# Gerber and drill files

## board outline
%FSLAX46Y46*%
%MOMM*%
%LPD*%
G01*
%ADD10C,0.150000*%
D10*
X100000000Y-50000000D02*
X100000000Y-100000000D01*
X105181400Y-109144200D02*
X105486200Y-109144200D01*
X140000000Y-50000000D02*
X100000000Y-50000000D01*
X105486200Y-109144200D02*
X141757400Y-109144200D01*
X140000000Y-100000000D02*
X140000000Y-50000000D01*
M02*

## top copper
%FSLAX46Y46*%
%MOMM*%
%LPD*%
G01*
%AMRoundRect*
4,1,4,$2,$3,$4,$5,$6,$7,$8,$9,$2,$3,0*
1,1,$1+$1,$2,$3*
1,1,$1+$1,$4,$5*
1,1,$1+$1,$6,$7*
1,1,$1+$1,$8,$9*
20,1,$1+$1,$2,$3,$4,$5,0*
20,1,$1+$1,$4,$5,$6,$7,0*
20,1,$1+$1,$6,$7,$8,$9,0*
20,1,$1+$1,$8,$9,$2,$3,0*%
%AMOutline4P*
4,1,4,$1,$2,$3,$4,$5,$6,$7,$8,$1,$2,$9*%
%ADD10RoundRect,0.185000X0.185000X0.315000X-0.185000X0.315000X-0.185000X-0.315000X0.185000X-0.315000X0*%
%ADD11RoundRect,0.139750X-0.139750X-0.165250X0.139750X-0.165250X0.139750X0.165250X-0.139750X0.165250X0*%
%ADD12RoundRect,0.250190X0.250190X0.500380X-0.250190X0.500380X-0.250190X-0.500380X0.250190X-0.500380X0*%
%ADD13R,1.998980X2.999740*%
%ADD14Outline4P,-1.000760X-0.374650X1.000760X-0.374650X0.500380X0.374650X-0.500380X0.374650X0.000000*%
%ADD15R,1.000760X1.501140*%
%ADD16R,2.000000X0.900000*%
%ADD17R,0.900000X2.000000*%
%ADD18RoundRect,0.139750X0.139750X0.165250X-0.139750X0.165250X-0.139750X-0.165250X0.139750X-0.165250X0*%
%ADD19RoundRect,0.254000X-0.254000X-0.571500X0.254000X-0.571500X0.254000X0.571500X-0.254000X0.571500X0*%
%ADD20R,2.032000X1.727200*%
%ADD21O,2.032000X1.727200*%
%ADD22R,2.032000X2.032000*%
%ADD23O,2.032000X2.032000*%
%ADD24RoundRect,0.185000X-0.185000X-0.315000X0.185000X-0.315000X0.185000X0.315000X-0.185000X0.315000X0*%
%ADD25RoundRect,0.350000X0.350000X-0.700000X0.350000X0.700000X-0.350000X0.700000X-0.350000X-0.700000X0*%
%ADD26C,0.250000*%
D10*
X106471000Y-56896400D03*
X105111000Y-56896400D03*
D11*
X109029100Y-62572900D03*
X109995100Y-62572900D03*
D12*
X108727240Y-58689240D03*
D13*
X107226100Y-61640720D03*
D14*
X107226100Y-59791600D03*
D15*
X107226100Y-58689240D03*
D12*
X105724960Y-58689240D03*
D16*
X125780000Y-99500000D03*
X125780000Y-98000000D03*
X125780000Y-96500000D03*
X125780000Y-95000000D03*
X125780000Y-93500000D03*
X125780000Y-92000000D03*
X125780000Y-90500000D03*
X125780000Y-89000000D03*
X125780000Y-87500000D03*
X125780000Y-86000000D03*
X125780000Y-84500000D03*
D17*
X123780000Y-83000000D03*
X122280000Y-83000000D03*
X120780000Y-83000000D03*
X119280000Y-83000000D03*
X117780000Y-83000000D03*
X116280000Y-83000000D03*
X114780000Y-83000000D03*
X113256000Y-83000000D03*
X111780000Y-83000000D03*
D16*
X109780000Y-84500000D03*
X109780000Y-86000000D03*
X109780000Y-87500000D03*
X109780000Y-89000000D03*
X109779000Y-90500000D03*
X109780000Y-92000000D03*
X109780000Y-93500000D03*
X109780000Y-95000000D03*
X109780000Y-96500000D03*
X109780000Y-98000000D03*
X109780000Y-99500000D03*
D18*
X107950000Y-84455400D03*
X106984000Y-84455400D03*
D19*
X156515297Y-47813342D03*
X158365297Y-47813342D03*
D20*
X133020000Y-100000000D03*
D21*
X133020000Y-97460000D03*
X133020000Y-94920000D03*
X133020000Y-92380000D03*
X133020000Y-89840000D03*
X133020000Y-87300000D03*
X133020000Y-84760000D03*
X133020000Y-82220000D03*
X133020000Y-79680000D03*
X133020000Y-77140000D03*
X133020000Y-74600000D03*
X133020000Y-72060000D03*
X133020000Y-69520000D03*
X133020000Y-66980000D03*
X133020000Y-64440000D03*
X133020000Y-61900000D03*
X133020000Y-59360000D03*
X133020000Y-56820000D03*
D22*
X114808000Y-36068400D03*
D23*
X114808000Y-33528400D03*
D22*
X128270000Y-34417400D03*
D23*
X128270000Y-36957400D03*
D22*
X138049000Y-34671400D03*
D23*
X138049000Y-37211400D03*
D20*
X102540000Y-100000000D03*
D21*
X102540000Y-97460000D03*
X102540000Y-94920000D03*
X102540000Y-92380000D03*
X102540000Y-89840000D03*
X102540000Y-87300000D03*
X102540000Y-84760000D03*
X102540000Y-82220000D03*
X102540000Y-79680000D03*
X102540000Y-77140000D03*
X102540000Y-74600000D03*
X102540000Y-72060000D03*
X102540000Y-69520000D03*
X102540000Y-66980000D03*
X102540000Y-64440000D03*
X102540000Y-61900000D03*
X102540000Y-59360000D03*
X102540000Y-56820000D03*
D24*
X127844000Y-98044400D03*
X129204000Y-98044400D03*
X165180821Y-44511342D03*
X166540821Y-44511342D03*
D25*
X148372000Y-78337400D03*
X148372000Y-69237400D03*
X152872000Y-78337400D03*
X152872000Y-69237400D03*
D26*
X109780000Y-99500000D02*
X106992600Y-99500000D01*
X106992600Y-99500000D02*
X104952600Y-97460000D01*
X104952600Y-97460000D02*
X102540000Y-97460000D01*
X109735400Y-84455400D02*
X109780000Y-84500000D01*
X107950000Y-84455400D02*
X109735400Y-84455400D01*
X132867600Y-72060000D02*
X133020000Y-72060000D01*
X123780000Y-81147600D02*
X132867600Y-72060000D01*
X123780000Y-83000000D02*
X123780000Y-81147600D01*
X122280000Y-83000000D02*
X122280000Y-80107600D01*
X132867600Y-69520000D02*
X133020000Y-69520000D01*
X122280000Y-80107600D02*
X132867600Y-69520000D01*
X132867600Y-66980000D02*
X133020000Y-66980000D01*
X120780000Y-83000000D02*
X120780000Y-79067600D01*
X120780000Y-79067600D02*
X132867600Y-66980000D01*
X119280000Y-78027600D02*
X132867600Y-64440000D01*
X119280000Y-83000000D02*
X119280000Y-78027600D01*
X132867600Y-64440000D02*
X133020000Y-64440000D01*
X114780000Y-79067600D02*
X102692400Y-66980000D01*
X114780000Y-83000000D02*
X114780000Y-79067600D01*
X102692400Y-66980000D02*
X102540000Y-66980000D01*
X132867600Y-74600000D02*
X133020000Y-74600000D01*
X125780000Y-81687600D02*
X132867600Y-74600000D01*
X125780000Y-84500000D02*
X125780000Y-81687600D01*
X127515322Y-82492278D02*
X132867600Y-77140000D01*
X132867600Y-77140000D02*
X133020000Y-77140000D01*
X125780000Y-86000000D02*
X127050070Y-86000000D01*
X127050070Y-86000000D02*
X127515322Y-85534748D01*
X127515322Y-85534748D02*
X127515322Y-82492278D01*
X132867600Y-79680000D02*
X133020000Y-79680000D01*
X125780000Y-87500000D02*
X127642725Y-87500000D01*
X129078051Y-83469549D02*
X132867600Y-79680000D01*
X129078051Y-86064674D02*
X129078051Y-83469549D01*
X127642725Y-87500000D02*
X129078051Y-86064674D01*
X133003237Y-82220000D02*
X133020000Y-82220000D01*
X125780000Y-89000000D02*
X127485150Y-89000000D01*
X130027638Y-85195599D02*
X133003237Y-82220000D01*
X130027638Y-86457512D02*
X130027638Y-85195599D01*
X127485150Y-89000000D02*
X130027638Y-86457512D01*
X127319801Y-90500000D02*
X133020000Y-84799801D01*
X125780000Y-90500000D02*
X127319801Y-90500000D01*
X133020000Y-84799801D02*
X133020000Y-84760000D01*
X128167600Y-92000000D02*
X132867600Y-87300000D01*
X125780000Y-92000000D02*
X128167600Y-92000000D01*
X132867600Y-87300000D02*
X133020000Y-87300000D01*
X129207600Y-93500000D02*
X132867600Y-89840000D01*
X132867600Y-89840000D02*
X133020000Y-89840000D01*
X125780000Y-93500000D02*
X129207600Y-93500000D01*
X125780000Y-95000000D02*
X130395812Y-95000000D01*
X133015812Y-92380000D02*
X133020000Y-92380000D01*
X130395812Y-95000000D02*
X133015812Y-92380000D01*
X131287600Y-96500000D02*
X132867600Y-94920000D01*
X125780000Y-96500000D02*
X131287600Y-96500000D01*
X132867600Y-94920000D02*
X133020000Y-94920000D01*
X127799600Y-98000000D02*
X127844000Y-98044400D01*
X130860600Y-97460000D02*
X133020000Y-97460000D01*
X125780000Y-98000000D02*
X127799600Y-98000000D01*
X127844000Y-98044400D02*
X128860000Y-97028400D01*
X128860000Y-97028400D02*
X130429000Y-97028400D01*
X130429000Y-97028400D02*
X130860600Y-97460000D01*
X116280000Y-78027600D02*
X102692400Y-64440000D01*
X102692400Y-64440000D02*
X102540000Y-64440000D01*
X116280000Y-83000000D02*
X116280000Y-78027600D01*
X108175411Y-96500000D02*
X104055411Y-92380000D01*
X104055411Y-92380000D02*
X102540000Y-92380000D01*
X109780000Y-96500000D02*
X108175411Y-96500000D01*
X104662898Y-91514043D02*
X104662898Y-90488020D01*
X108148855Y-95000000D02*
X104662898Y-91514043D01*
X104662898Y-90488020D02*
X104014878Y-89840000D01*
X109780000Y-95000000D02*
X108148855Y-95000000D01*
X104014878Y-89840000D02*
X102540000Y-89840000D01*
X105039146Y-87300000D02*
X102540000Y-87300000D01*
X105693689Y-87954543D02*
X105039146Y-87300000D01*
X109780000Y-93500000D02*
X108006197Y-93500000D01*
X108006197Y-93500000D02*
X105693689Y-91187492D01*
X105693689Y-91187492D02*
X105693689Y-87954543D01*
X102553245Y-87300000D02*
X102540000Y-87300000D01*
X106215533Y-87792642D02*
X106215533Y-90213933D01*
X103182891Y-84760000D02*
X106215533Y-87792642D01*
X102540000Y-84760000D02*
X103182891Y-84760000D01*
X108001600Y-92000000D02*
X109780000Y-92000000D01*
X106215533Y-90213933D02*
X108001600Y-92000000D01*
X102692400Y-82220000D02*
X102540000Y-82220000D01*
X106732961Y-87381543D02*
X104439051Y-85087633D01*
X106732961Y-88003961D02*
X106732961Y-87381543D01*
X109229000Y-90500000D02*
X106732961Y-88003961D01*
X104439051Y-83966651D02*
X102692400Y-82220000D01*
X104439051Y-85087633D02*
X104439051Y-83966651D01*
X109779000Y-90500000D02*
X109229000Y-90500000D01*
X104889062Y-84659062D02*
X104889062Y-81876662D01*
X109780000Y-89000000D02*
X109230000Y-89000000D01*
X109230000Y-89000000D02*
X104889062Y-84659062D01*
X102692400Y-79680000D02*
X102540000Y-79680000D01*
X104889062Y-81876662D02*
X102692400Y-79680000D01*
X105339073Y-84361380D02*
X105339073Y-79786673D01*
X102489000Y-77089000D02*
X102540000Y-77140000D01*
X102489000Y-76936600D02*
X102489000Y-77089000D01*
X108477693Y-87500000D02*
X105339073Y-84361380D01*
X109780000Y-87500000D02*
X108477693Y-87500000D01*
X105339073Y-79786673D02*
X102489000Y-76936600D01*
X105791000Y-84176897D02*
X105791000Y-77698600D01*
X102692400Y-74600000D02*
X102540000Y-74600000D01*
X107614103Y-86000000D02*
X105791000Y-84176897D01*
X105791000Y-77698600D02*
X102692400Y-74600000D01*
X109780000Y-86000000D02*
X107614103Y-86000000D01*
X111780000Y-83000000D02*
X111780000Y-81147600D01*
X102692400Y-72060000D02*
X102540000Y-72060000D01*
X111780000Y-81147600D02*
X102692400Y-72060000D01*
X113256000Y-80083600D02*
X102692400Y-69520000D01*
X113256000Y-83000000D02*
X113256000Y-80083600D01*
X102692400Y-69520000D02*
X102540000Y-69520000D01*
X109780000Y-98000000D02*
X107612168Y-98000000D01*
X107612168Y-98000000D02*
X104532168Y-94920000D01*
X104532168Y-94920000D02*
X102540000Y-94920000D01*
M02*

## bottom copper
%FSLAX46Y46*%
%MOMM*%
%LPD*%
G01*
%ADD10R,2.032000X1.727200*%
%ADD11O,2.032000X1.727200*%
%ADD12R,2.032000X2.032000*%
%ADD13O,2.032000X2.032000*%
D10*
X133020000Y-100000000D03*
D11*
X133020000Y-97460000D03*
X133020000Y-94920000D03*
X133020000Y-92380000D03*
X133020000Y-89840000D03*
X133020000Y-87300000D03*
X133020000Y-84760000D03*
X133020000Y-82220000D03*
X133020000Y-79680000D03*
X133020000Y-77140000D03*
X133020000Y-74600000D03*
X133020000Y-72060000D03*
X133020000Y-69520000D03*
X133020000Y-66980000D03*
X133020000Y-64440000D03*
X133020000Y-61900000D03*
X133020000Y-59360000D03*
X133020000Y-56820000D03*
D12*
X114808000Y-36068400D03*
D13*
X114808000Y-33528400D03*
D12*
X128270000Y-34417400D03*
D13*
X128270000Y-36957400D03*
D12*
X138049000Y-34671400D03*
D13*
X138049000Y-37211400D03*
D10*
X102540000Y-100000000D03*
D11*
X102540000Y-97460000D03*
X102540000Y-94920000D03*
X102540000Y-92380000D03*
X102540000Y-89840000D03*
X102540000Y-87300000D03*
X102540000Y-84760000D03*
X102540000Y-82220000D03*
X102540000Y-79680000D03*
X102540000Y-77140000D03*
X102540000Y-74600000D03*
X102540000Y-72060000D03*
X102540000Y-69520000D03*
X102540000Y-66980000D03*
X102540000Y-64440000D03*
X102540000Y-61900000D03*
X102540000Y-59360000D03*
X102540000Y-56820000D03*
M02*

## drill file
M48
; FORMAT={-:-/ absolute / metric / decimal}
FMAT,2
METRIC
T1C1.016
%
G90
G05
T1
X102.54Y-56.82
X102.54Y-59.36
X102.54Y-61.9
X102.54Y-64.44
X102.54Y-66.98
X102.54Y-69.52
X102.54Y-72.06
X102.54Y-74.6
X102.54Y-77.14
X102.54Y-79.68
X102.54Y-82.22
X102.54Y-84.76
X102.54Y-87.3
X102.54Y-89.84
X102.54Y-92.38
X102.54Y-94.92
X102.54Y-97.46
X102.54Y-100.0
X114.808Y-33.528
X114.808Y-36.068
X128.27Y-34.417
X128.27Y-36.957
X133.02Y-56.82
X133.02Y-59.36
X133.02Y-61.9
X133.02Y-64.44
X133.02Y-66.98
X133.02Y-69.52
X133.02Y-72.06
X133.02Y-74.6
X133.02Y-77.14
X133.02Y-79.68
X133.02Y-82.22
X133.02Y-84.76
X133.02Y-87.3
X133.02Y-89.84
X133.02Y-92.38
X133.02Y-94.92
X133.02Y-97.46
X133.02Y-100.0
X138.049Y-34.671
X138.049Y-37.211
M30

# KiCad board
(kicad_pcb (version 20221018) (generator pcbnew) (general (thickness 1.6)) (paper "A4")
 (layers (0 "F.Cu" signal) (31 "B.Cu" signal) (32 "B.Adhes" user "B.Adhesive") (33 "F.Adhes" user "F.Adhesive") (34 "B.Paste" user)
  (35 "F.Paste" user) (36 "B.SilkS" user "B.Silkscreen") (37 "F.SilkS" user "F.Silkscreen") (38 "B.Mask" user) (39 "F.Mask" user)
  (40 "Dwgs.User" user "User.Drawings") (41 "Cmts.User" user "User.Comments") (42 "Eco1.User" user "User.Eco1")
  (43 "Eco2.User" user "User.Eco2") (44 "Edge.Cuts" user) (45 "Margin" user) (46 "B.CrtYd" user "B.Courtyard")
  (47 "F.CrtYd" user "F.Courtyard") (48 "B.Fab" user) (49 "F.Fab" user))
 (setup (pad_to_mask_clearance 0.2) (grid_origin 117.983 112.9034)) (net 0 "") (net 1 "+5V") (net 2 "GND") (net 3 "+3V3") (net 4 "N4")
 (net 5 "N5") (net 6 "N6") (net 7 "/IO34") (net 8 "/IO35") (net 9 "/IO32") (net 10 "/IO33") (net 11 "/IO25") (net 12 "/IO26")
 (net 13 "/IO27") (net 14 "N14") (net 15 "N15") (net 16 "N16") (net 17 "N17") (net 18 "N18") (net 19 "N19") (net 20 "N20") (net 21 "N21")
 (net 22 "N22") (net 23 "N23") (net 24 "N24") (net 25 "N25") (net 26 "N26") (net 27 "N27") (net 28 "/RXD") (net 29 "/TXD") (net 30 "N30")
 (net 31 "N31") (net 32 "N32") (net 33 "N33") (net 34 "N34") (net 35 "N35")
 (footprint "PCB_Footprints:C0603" (layer "F.Cu") (at 105.791 56.8964 180)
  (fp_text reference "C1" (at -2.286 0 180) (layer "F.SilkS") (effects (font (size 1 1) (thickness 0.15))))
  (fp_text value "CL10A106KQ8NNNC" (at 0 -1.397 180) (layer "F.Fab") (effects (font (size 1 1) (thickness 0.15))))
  (pad "1" smd roundrect (at -0.68 0 180) (size 0.74 1) (layers "F.Cu" "F.Paste" "F.Mask") (roundrect_rratio 0.25) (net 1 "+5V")
   (solder_mask_margin 0.102))
  (pad "2" smd roundrect (at 0.68 0 180) (size 0.74 1) (layers "F.Cu" "F.Paste" "F.Mask") (roundrect_rratio 0.25) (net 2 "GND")
   (solder_mask_margin 0.102)))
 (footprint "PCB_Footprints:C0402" (layer "F.Cu") (at 109.5121 62.5729)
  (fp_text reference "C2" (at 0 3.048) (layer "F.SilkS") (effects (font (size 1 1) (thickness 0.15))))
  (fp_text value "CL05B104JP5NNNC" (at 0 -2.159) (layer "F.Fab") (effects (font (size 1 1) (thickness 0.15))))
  (pad "1" smd roundrect (at -0.483 0) (size 0.559 0.61) (layers "F.Cu" "F.Paste" "F.Mask") (roundrect_rratio 0.25) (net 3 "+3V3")
   (solder_mask_margin 0.102))
  (pad "2" smd roundrect (at 0.483 0) (size 0.559 0.61) (layers "F.Cu" "F.Paste" "F.Mask") (roundrect_rratio 0.25) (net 2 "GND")
   (solder_mask_margin 0.102)))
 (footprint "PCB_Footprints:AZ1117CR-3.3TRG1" (layer "F.Cu") (at 107.2261 60.5409 180)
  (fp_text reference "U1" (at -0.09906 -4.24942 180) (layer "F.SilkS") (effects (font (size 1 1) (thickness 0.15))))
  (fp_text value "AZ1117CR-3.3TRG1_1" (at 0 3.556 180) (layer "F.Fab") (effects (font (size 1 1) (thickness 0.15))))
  (pad "1" smd roundrect (at -1.50114 1.85166 180) (size 1.00076 1.50114) (layers "F.Cu" "F.Paste" "F.Mask") (roundrect_rratio 0.25)
   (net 2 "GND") (solder_mask_margin 0.102))
  (pad "2" smd rect (at 0 -1.09982 180) (size 1.99898 2.99974) (layers "F.Cu" "F.Paste" "F.Mask") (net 3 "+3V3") (solder_mask_margin 0.102))
  (pad "2" smd trapezoid (at 0 0.7493) (size 1.50114 0.7493) (rect_delta 0 0.50038) (layers "F.Cu" "F.Paste" "F.Mask") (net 3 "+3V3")
   (solder_mask_margin 0.102))
  (pad "2" smd rect (at 0 1.85166 180) (size 1.00076 1.50114) (layers "F.Cu" "F.Paste" "F.Mask") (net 3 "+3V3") (solder_mask_margin 0.102))
  (pad "3" smd roundrect (at 1.50114 1.85166 180) (size 1.00076 1.50114) (layers "F.Cu" "F.Paste" "F.Mask") (roundrect_rratio 0.25)
   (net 1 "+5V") (solder_mask_margin 0.102)))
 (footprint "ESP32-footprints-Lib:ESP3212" (layer "F.Cu") (at 117.78 95 180)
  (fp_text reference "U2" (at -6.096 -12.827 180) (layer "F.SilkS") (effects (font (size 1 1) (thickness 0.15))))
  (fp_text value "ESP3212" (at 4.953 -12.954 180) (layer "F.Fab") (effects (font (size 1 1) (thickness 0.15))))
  (pad "1" smd rect (at -8 -4.5 180) (size 2 0.9) (layers "F.Cu" "F.Paste" "F.Mask") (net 2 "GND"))
  (pad "2" smd rect (at -8 -3 180) (size 2 0.9) (layers "F.Cu" "F.Paste" "F.Mask") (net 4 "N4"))
  (pad "3" smd rect (at -8 -1.5 180) (size 2 0.9) (layers "F.Cu" "F.Paste" "F.Mask") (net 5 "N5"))
  (pad "4" smd rect (at -8 0 180) (size 2 0.9) (layers "F.Cu" "F.Paste" "F.Mask") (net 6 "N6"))
  (pad "5" smd rect (at -8 1.5 180) (size 2 0.9) (layers "F.Cu" "F.Paste" "F.Mask") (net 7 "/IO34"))
  (pad "6" smd rect (at -8 3 180) (size 2 0.9) (layers "F.Cu" "F.Paste" "F.Mask") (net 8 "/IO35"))
  (pad "7" smd rect (at -8 4.5 180) (size 2 0.9) (layers "F.Cu" "F.Paste" "F.Mask") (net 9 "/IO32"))
  (pad "8" smd rect (at -8 6 180) (size 2 0.9) (layers "F.Cu" "F.Paste" "F.Mask") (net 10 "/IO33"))
  (pad "9" smd rect (at -8 7.5 180) (size 2 0.9) (layers "F.Cu" "F.Paste" "F.Mask") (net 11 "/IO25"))
  (pad "10" smd rect (at -8 9 180) (size 2 0.9) (layers "F.Cu" "F.Paste" "F.Mask") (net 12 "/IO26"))
  (pad "11" smd rect (at -8 10.5 180) (size 2 0.9) (layers "F.Cu" "F.Paste" "F.Mask") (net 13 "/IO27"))
  (pad "12" smd rect (at -6 12 180) (size 0.9 2) (layers "F.Cu" "F.Paste" "F.Mask") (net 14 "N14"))
  (pad "13" smd rect (at -4.5 12 180) (size 0.9 2) (layers "F.Cu" "F.Paste" "F.Mask") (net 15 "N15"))
  (pad "14" smd rect (at -3 12 180) (size 0.9 2) (layers "F.Cu" "F.Paste" "F.Mask") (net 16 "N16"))
  (pad "15" smd rect (at -1.5 12 180) (size 0.9 2) (layers "F.Cu" "F.Paste" "F.Mask") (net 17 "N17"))
  (pad "16" smd rect (at 0 12 180) (size 0.9 2) (layers "F.Cu" "F.Paste" "F.Mask") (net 2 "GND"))
  (pad "17" smd rect (at 1.5 12 180) (size 0.9 2) (layers "F.Cu" "F.Paste" "F.Mask") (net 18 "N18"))
  (pad "18" smd rect (at 3 12 180) (size 0.9 2) (layers "F.Cu" "F.Paste" "F.Mask") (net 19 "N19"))
  (pad "19" smd rect (at 4.524 12 180) (size 0.9 2) (layers "F.Cu" "F.Paste" "F.Mask") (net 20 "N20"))
  (pad "20" smd rect (at 6 12 180) (size 0.9 2) (layers "F.Cu" "F.Paste" "F.Mask") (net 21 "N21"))
  (pad "21" smd rect (at 8 10.5 180) (size 2 0.9) (layers "F.Cu" "F.Paste" "F.Mask") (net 3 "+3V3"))
  (pad "22" smd rect (at 8 9 180) (size 2 0.9) (layers "F.Cu" "F.Paste" "F.Mask") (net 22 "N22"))
  (pad "23" smd rect (at 8 7.5 180) (size 2 0.9) (layers "F.Cu" "F.Paste" "F.Mask") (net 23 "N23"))
  (pad "24" smd rect (at 8 6 180) (size 2 0.9) (layers "F.Cu" "F.Paste" "F.Mask") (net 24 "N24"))
  (pad "25" smd rect (at 8.001 4.5 180) (size 2 0.9) (layers "F.Cu" "F.Paste" "F.Mask") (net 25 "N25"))
  (pad "26" smd rect (at 8 3 180) (size 2 0.9) (layers "F.Cu" "F.Paste" "F.Mask") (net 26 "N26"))
  (pad "27" smd rect (at 8 1.5 180) (size 2 0.9) (layers "F.Cu" "F.Paste" "F.Mask") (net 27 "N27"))
  (pad "28" smd rect (at 8 0 180) (size 2 0.9) (layers "F.Cu" "F.Paste" "F.Mask") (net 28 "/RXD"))
  (pad "29" smd rect (at 8 -1.5 180) (size 2 0.9) (layers "F.Cu" "F.Paste" "F.Mask") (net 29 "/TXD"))
  (pad "30" smd rect (at 8 -3 180) (size 2 0.9) (layers "F.Cu" "F.Paste" "F.Mask") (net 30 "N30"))
  (pad "31" smd rect (at 8 -4.5 180) (size 2 0.9) (layers "F.Cu" "F.Paste" "F.Mask") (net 2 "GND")))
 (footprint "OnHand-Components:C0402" (layer "F.Cu") (at 107.467 84.4554 180)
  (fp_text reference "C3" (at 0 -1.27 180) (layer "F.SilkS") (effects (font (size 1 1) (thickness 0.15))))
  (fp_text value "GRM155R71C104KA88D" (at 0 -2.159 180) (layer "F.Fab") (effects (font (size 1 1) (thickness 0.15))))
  (pad "1" smd roundrect (at -0.483 0 180) (size 0.559 0.61) (layers "F.Cu" "F.Paste" "F.Mask") (roundrect_rratio 0.25) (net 3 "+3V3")
   (solder_mask_margin 0.102))
  (pad "2" smd roundrect (at 0.483 0 180) (size 0.559 0.61) (layers "F.Cu" "F.Paste" "F.Mask") (roundrect_rratio 0.25) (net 2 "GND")
   (solder_mask_margin 0.102)))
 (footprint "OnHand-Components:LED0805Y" (layer "F.Cu") (at 157.440297 47.813342)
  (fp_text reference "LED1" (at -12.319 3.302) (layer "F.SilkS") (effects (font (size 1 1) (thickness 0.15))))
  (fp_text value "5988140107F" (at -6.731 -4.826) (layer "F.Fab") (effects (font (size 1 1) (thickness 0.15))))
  (pad "1" smd roundrect (at -0.925 0) (size 1.016 1.651) (layers "F.Cu" "F.Paste" "F.Mask") (roundrect_rratio 0.25) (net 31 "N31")
   (solder_mask_margin 0.102))
  (pad "2" smd roundrect (at 0.925 0) (size 1.016 1.651) (layers "F.Cu" "F.Paste" "F.Mask") (roundrect_rratio 0.25) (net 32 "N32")
   (solder_mask_margin 0.102)))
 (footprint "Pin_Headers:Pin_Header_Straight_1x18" (layer "F.Cu") (at 133.02 100 180)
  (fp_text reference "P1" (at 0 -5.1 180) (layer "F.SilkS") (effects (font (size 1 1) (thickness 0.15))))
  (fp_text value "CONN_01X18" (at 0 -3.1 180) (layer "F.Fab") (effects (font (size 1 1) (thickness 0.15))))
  (pad "1" thru_hole rect (at 0 0 180) (size 2.032 1.7272) (drill 1.016) (layers "*.Cu" "*.Mask" "F.SilkS") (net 2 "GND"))
  (pad "2" thru_hole oval (at 0 2.54 180) (size 2.032 1.7272) (drill 1.016) (layers "*.Cu" "*.Mask" "F.SilkS") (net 4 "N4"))
  (pad "3" thru_hole oval (at 0 5.08 180) (size 2.032 1.7272) (drill 1.016) (layers "*.Cu" "*.Mask" "F.SilkS") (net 5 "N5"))
  (pad "4" thru_hole oval (at 0 7.62 180) (size 2.032 1.7272) (drill 1.016) (layers "*.Cu" "*.Mask" "F.SilkS") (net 6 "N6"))
  (pad "5" thru_hole oval (at 0 10.16 180) (size 2.032 1.7272) (drill 1.016) (layers "*.Cu" "*.Mask" "F.SilkS") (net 7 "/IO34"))
  (pad "6" thru_hole oval (at 0 12.7 180) (size 2.032 1.7272) (drill 1.016) (layers "*.Cu" "*.Mask" "F.SilkS") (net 8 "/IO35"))
  (pad "7" thru_hole oval (at 0 15.24 180) (size 2.032 1.7272) (drill 1.016) (layers "*.Cu" "*.Mask" "F.SilkS") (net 9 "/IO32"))
  (pad "8" thru_hole oval (at 0 17.78 180) (size 2.032 1.7272) (drill 1.016) (layers "*.Cu" "*.Mask" "F.SilkS") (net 10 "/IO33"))
  (pad "9" thru_hole oval (at 0 20.32 180) (size 2.032 1.7272) (drill 1.016) (layers "*.Cu" "*.Mask" "F.SilkS") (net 11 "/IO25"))
  (pad "10" thru_hole oval (at 0 22.86 180) (size 2.032 1.7272) (drill 1.016) (layers "*.Cu" "*.Mask" "F.SilkS") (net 12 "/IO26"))
  (pad "11" thru_hole oval (at 0 25.4 180) (size 2.032 1.7272) (drill 1.016) (layers "*.Cu" "*.Mask" "F.SilkS") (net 13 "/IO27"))
  (pad "12" thru_hole oval (at 0 27.94 180) (size 2.032 1.7272) (drill 1.016) (layers "*.Cu" "*.Mask" "F.SilkS") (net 14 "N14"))
  (pad "13" thru_hole oval (at 0 30.48 180) (size 2.032 1.7272) (drill 1.016) (layers "*.Cu" "*.Mask" "F.SilkS") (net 15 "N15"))
  (pad "14" thru_hole oval (at 0 33.02 180) (size 2.032 1.7272) (drill 1.016) (layers "*.Cu" "*.Mask" "F.SilkS") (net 16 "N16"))
  (pad "15" thru_hole oval (at 0 35.56 180) (size 2.032 1.7272) (drill 1.016) (layers "*.Cu" "*.Mask" "F.SilkS") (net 17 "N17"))
  (pad "16" thru_hole oval (at 0 38.1 180) (size 2.032 1.7272) (drill 1.016) (layers "*.Cu" "*.Mask" "F.SilkS") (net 3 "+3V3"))
  (pad "17" thru_hole oval (at 0 40.64 180) (size 2.032 1.7272) (drill 1.016) (layers "*.Cu" "*.Mask" "F.SilkS") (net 1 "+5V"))
  (pad "18" thru_hole oval (at 0 43.18 180) (size 2.032 1.7272) (drill 1.016) (layers "*.Cu" "*.Mask" "F.SilkS") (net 2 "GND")))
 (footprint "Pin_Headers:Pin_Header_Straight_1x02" (layer "F.Cu") (at 114.808 36.0684 180)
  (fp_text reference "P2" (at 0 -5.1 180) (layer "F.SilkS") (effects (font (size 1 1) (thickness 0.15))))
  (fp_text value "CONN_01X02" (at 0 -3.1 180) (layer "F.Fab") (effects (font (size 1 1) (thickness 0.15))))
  (pad "1" thru_hole rect (at 0 0 180) (size 2.032 2.032) (drill 1.016) (layers "*.Cu" "*.Mask" "F.SilkS") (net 19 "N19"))
  (pad "2" thru_hole oval (at 0 2.54 180) (size 2.032 2.032) (drill 1.016) (layers "*.Cu" "*.Mask" "F.SilkS") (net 2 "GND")))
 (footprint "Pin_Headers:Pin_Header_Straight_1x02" (layer "F.Cu") (at 128.27 34.4174)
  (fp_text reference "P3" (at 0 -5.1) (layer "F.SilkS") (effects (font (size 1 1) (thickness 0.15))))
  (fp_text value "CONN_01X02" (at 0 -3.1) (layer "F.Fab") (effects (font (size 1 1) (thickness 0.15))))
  (pad "1" thru_hole rect (at 0 0) (size 2.032 2.032) (drill 1.016) (layers "*.Cu" "*.Mask" "F.SilkS") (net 18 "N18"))
  (pad "2" thru_hole oval (at 0 2.54) (size 2.032 2.032) (drill 1.016) (layers "*.Cu" "*.Mask" "F.SilkS") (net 2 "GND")))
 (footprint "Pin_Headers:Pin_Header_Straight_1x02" (layer "F.Cu") (at 138.049 34.6714)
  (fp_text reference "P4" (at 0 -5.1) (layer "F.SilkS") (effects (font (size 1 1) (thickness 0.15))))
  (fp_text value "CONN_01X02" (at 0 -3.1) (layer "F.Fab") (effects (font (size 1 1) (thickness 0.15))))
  (pad "1" thru_hole rect (at 0 0) (size 2.032 2.032) (drill 1.016) (layers "*.Cu" "*.Mask" "F.SilkS") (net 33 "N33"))
  (pad "2" thru_hole oval (at 0 2.54) (size 2.032 2.032) (drill 1.016) (layers "*.Cu" "*.Mask" "F.SilkS") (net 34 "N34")))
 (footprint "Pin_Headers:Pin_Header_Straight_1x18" (layer "F.Cu") (at 102.54 100 180)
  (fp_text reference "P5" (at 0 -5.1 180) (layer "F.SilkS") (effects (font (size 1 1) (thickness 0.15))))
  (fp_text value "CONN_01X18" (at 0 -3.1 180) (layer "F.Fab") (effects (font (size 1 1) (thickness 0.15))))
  (pad "1" thru_hole rect (at 0 0 180) (size 2.032 1.7272) (drill 1.016) (layers "*.Cu" "*.Mask" "F.SilkS") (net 2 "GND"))
  (pad "2" thru_hole oval (at 0 2.54 180) (size 2.032 1.7272) (drill 1.016) (layers "*.Cu" "*.Mask" "F.SilkS") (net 2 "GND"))
  (pad "3" thru_hole oval (at 0 5.08 180) (size 2.032 1.7272) (drill 1.016) (layers "*.Cu" "*.Mask" "F.SilkS") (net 30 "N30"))
  (pad "4" thru_hole oval (at 0 7.62 180) (size 2.032 1.7272) (drill 1.016) (layers "*.Cu" "*.Mask" "F.SilkS") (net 29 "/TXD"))
  (pad "5" thru_hole oval (at 0 10.16 180) (size 2.032 1.7272) (drill 1.016) (layers "*.Cu" "*.Mask" "F.SilkS") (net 28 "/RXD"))
  (pad "6" thru_hole oval (at 0 12.7 180) (size 2.032 1.7272) (drill 1.016) (layers "*.Cu" "*.Mask" "F.SilkS") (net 27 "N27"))
  (pad "7" thru_hole oval (at 0 15.24 180) (size 2.032 1.7272) (drill 1.016) (layers "*.Cu" "*.Mask" "F.SilkS") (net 26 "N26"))
  (pad "8" thru_hole oval (at 0 17.78 180) (size 2.032 1.7272) (drill 1.016) (layers "*.Cu" "*.Mask" "F.SilkS") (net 25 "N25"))
  (pad "9" thru_hole oval (at 0 20.32 180) (size 2.032 1.7272) (drill 1.016) (layers "*.Cu" "*.Mask" "F.SilkS") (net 24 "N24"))
  (pad "10" thru_hole oval (at 0 22.86 180) (size 2.032 1.7272) (drill 1.016) (layers "*.Cu" "*.Mask" "F.SilkS") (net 23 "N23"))
  (pad "11" thru_hole oval (at 0 25.4 180) (size 2.032 1.7272) (drill 1.016) (layers "*.Cu" "*.Mask" "F.SilkS") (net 22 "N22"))
  (pad "12" thru_hole oval (at 0 27.94 180) (size 2.032 1.7272) (drill 1.016) (layers "*.Cu" "*.Mask" "F.SilkS") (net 21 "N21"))
  (pad "13" thru_hole oval (at 0 30.48 180) (size 2.032 1.7272) (drill 1.016) (layers "*.Cu" "*.Mask" "F.SilkS") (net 20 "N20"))
  (pad "14" thru_hole oval (at 0 33.02 180) (size 2.032 1.7272) (drill 1.016) (layers "*.Cu" "*.Mask" "F.SilkS") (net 19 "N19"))
  (pad "15" thru_hole oval (at 0 35.56 180) (size 2.032 1.7272) (drill 1.016) (layers "*.Cu" "*.Mask" "F.SilkS") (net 18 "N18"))
  (pad "16" thru_hole oval (at 0 38.1 180) (size 2.032 1.7272) (drill 1.016) (layers "*.Cu" "*.Mask" "F.SilkS") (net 3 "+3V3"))
  (pad "17" thru_hole oval (at 0 40.64 180) (size 2.032 1.7272) (drill 1.016) (layers "*.Cu" "*.Mask" "F.SilkS") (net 1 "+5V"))
  (pad "18" thru_hole oval (at 0 43.18 180) (size 2.032 1.7272) (drill 1.016) (layers "*.Cu" "*.Mask" "F.SilkS") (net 2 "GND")))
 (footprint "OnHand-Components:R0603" (layer "F.Cu") (at 128.524 98.0444)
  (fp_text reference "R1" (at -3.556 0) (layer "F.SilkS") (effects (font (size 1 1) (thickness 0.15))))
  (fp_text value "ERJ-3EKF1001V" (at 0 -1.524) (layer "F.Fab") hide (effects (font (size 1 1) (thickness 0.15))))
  (pad "1" smd roundrect (at -0.68 0) (size 0.74 1) (layers "F.Cu" "F.Paste" "F.Mask") (roundrect_rratio 0.25) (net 4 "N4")
   (solder_mask_margin 0.102))
  (pad "2" smd roundrect (at 0.68 0) (size 0.74 1) (layers "F.Cu" "F.Paste" "F.Mask") (roundrect_rratio 0.25) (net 3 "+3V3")
   (solder_mask_margin 0.102)))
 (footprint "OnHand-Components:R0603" (layer "F.Cu") (at 165.860821 44.511342)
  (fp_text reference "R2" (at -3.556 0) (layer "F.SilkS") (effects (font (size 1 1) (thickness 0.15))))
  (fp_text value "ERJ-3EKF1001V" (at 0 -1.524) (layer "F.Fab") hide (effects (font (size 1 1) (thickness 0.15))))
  (pad "1" smd roundrect (at -0.68 0) (size 0.74 1) (layers "F.Cu" "F.Paste" "F.Mask") (roundrect_rratio 0.25) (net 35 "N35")
   (solder_mask_margin 0.102))
  (pad "2" smd roundrect (at 0.68 0) (size 0.74 1) (layers "F.Cu" "F.Paste" "F.Mask") (roundrect_rratio 0.25) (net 33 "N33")
   (solder_mask_margin 0.102)))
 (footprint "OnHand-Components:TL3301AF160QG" (layer "F.Cu") (at 150.622 73.7874 90)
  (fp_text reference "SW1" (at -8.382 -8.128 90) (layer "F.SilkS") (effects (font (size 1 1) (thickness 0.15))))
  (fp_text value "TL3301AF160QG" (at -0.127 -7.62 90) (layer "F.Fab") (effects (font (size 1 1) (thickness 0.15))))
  (pad "1" smd roundrect (at -4.55 -2.25 90) (size 2.1 1.4) (layers "F.Cu" "F.Paste" "F.Mask") (roundrect_rratio 0.25) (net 2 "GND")
   (solder_mask_margin 0.102))
  (pad "1" smd roundrect (at 4.55 -2.25 90) (size 2.1 1.4) (layers "F.Cu" "F.Paste" "F.Mask") (roundrect_rratio 0.25) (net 2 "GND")
   (solder_mask_margin 0.102))
  (pad "2" smd roundrect (at -4.55 2.25 90) (size 2.1 1.4) (layers "F.Cu" "F.Paste" "F.Mask") (roundrect_rratio 0.25) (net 4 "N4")
   (solder_mask_margin 0.102))
  (pad "2" smd roundrect (at 4.55 2.25 90) (size 2.1 1.4) (layers "F.Cu" "F.Paste" "F.Mask") (roundrect_rratio 0.25) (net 4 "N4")
   (solder_mask_margin 0.102)))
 (gr_line (start 100 50) (end 100 100) (stroke (width 0.15) (type solid)) (layer "Edge.Cuts"))
 (gr_line (start 105.1814 109.1442) (end 105.4862 109.1442) (stroke (width 0.15) (type solid)) (layer "Edge.Cuts"))
 (gr_line (start 140 50) (end 100 50) (stroke (width 0.15) (type solid)) (layer "Edge.Cuts"))
 (gr_line (start 105.4862 109.1442) (end 141.7574 109.1442) (stroke (width 0.15) (type solid)) (layer "Edge.Cuts"))
 (gr_line (start 140 100) (end 140 50) (stroke (width 0.15) (type solid)) (layer "Edge.Cuts"))
 (segment (start 109.78 99.5) (end 106.9926 99.5) (width 0.25) (layer "F.Cu") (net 2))
 (segment (start 106.9926 99.5) (end 104.9526 97.46) (width 0.25) (layer "F.Cu") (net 2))
 (segment (start 104.9526 97.46) (end 102.54 97.46) (width 0.25) (layer "F.Cu") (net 2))
 (segment (start 109.7354 84.4554) (end 109.78 84.5) (width 0.25) (layer "F.Cu") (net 3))
 (segment (start 107.95 84.4554) (end 109.7354 84.4554) (width 0.25) (layer "F.Cu") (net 3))
 (segment (start 132.8676 72.06) (end 133.02 72.06) (width 0.25) (layer "F.Cu") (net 14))
 (segment (start 123.78 81.1476) (end 132.8676 72.06) (width 0.25) (layer "F.Cu") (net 14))
 (segment (start 123.78 83) (end 123.78 81.1476) (width 0.25) (layer "F.Cu") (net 14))
 (segment (start 122.28 83) (end 122.28 80.1076) (width 0.25) (layer "F.Cu") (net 15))
 (segment (start 132.8676 69.52) (end 133.02 69.52) (width 0.25) (layer "F.Cu") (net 15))
 (segment (start 122.28 80.1076) (end 132.8676 69.52) (width 0.25) (layer "F.Cu") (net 15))
 (segment (start 132.8676 66.98) (end 133.02 66.98) (width 0.25) (layer "F.Cu") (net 16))
 (segment (start 120.78 83) (end 120.78 79.0676) (width 0.25) (layer "F.Cu") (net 16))
 (segment (start 120.78 79.0676) (end 132.8676 66.98) (width 0.25) (layer "F.Cu") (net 16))
 (segment (start 119.28 78.0276) (end 132.8676 64.44) (width 0.25) (layer "F.Cu") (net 17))
 (segment (start 119.28 83) (end 119.28 78.0276) (width 0.25) (layer "F.Cu") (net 17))
 (segment (start 132.8676 64.44) (end 133.02 64.44) (width 0.25) (layer "F.Cu") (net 17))
 (segment (start 114.78 79.0676) (end 102.6924 66.98) (width 0.25) (layer "F.Cu") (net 19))
 (segment (start 114.78 83) (end 114.78 79.0676) (width 0.25) (layer "F.Cu") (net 19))
 (segment (start 102.6924 66.98) (end 102.54 66.98) (width 0.25) (layer "F.Cu") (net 19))
 (segment (start 132.8676 74.6) (end 133.02 74.6) (width 0.25) (layer "F.Cu") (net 13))
 (segment (start 125.78 81.6876) (end 132.8676 74.6) (width 0.25) (layer "F.Cu") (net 13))
 (segment (start 125.78 84.5) (end 125.78 81.6876) (width 0.25) (layer "F.Cu") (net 13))
 (segment (start 127.515322 82.492278) (end 132.8676 77.14) (width 0.25) (layer "F.Cu") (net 12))
 (segment (start 132.8676 77.14) (end 133.02 77.14) (width 0.25) (layer "F.Cu") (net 12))
 (segment (start 125.78 86) (end 127.05007 86) (width 0.25) (layer "F.Cu") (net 12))
 (segment (start 127.05007 86) (end 127.515322 85.534748) (width 0.25) (layer "F.Cu") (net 12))
 (segment (start 127.515322 85.534748) (end 127.515322 82.492278) (width 0.25) (layer "F.Cu") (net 12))
 (segment (start 132.8676 79.68) (end 133.02 79.68) (width 0.25) (layer "F.Cu") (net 11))
 (segment (start 125.78 87.5) (end 127.642725 87.5) (width 0.25) (layer "F.Cu") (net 11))
 (segment (start 129.078051 83.469549) (end 132.8676 79.68) (width 0.25) (layer "F.Cu") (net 11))
 (segment (start 129.078051 86.064674) (end 129.078051 83.469549) (width 0.25) (layer "F.Cu") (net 11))
 (segment (start 127.642725 87.5) (end 129.078051 86.064674) (width 0.25) (layer "F.Cu") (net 11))
 (segment (start 133.003237 82.22) (end 133.02 82.22) (width 0.25) (layer "F.Cu") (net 10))
 (segment (start 125.78 89) (end 127.48515 89) (width 0.25) (layer "F.Cu") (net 10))
 (segment (start 130.027638 85.195599) (end 133.003237 82.22) (width 0.25) (layer "F.Cu") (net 10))
 (segment (start 130.027638 86.457512) (end 130.027638 85.195599) (width 0.25) (layer "F.Cu") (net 10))
 (segment (start 127.48515 89) (end 130.027638 86.457512) (width 0.25) (layer "F.Cu") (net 10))
 (segment (start 127.319801 90.5) (end 133.02 84.799801) (width 0.25) (layer "F.Cu") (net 9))
 (segment (start 125.78 90.5) (end 127.319801 90.5) (width 0.25) (layer "F.Cu") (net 9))
 (segment (start 133.02 84.799801) (end 133.02 84.76) (width 0.25) (layer "F.Cu") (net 9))
 (segment (start 128.1676 92) (end 132.8676 87.3) (width 0.25) (layer "F.Cu") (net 8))
 (segment (start 125.78 92) (end 128.1676 92) (width 0.25) (layer "F.Cu") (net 8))
 (segment (start 132.8676 87.3) (end 133.02 87.3) (width 0.25) (layer "F.Cu") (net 8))
 (segment (start 129.2076 93.5) (end 132.8676 89.84) (width 0.25) (layer "F.Cu") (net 7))
 (segment (start 132.8676 89.84) (end 133.02 89.84) (width 0.25) (layer "F.Cu") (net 7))
 (segment (start 125.78 93.5) (end 129.2076 93.5) (width 0.25) (layer "F.Cu") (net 7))
 (segment (start 125.78 95) (end 130.395812 95) (width 0.25) (layer "F.Cu") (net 6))
 (segment (start 133.015812 92.38) (end 133.02 92.38) (width 0.25) (layer "F.Cu") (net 6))
 (segment (start 130.395812 95) (end 133.015812 92.38) (width 0.25) (layer "F.Cu") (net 6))
 (segment (start 131.2876 96.5) (end 132.8676 94.92) (width 0.25) (layer "F.Cu") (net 5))
 (segment (start 125.78 96.5) (end 131.2876 96.5) (width 0.25) (layer "F.Cu") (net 5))
 (segment (start 132.8676 94.92) (end 133.02 94.92) (width 0.25) (layer "F.Cu") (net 5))
 (segment (start 127.7996 98) (end 127.844 98.0444) (width 0.25) (layer "F.Cu") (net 4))
 (segment (start 130.8606 97.46) (end 133.02 97.46) (width 0.25) (layer "F.Cu") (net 4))
 (segment (start 125.78 98) (end 127.7996 98) (width 0.25) (layer "F.Cu") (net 4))
 (segment (start 127.844 98.0444) (end 128.86 97.0284) (width 0.25) (layer "F.Cu") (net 4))
 (segment (start 128.86 97.0284) (end 130.429 97.0284) (width 0.25) (layer "F.Cu") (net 4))
 (segment (start 130.429 97.0284) (end 130.8606 97.46) (width 0.25) (layer "F.Cu") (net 4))
 (segment (start 116.28 78.0276) (end 102.6924 64.44) (width 0.25) (layer "F.Cu") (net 18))
 (segment (start 102.6924 64.44) (end 102.54 64.44) (width 0.25) (layer "F.Cu") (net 18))
 (segment (start 116.28 83) (end 116.28 78.0276) (width 0.25) (layer "F.Cu") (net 18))
 (segment (start 108.175411 96.5) (end 104.055411 92.38) (width 0.25) (layer "F.Cu") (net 29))
 (segment (start 104.055411 92.38) (end 102.54 92.38) (width 0.25) (layer "F.Cu") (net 29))
 (segment (start 109.78 96.5) (end 108.175411 96.5) (width 0.25) (layer "F.Cu") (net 29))
 (segment (start 104.662898 91.514043) (end 104.662898 90.48802) (width 0.25) (layer "F.Cu") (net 28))
 (segment (start 108.148855 95) (end 104.662898 91.514043) (width 0.25) (layer "F.Cu") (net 28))
 (segment (start 104.662898 90.48802) (end 104.014878 89.84) (width 0.25) (layer "F.Cu") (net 28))
 (segment (start 109.78 95) (end 108.148855 95) (width 0.25) (layer "F.Cu") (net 28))
 (segment (start 104.014878 89.84) (end 102.54 89.84) (width 0.25) (layer "F.Cu") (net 28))
 (segment (start 105.039146 87.3) (end 102.54 87.3) (width 0.25) (layer "F.Cu") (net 27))
 (segment (start 105.693689 87.954543) (end 105.039146 87.3) (width 0.25) (layer "F.Cu") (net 27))
 (segment (start 109.78 93.5) (end 108.006197 93.5) (width 0.25) (layer "F.Cu") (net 27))
 (segment (start 108.006197 93.5) (end 105.693689 91.187492) (width 0.25) (layer "F.Cu") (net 27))
 (segment (start 105.693689 91.187492) (end 105.693689 87.954543) (width 0.25) (layer "F.Cu") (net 27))
 (segment (start 102.553245 87.3) (end 102.54 87.3) (width 0.25) (layer "F.Cu") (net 27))
 (segment (start 106.215533 87.792642) (end 106.215533 90.213933) (width 0.25) (layer "F.Cu") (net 26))
 (segment (start 103.182891 84.76) (end 106.215533 87.792642) (width 0.25) (layer "F.Cu") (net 26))
 (segment (start 102.54 84.76) (end 103.182891 84.76) (width 0.25) (layer "F.Cu") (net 26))
 (segment (start 108.0016 92) (end 109.78 92) (width 0.25) (layer "F.Cu") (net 26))
 (segment (start 106.215533 90.213933) (end 108.0016 92) (width 0.25) (layer "F.Cu") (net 26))
 (segment (start 102.6924 82.22) (end 102.54 82.22) (width 0.25) (layer "F.Cu") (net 25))
 (segment (start 106.732961 87.381543) (end 104.439051 85.087633) (width 0.25) (layer "F.Cu") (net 25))
 (segment (start 106.732961 88.003961) (end 106.732961 87.381543) (width 0.25) (layer "F.Cu") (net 25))
 (segment (start 109.229 90.5) (end 106.732961 88.003961) (width 0.25) (layer "F.Cu") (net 25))
 (segment (start 104.439051 83.966651) (end 102.6924 82.22) (width 0.25) (layer "F.Cu") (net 25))
 (segment (start 104.439051 85.087633) (end 104.439051 83.966651) (width 0.25) (layer "F.Cu") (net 25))
 (segment (start 109.779 90.5) (end 109.229 90.5) (width 0.25) (layer "F.Cu") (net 25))
 (segment (start 104.889062 84.659062) (end 104.889062 81.876662) (width 0.25) (layer "F.Cu") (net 24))
 (segment (start 109.78 89) (end 109.23 89) (width 0.25) (layer "F.Cu") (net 24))
 (segment (start 109.23 89) (end 104.889062 84.659062) (width 0.25) (layer "F.Cu") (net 24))
 (segment (start 102.6924 79.68) (end 102.54 79.68) (width 0.25) (layer "F.Cu") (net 24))
 (segment (start 104.889062 81.876662) (end 102.6924 79.68) (width 0.25) (layer "F.Cu") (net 24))
 (segment (start 105.339073 84.36138) (end 105.339073 79.786673) (width 0.25) (layer "F.Cu") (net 23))
 (segment (start 102.489 77.089) (end 102.54 77.14) (width 0.25) (layer "F.Cu") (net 23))
 (segment (start 102.489 76.9366) (end 102.489 77.089) (width 0.25) (layer "F.Cu") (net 23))
 (segment (start 108.477693 87.5) (end 105.339073 84.36138) (width 0.25) (layer "F.Cu") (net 23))
 (segment (start 109.78 87.5) (end 108.477693 87.5) (width 0.25) (layer "F.Cu") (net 23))
 (segment (start 105.339073 79.786673) (end 102.489 76.9366) (width 0.25) (layer "F.Cu") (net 23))
 (segment (start 105.791 84.176897) (end 105.791 77.6986) (width 0.25) (layer "F.Cu") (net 22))
 (segment (start 102.6924 74.6) (end 102.54 74.6) (width 0.25) (layer "F.Cu") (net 22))
 (segment (start 107.614103 86) (end 105.791 84.176897) (width 0.25) (layer "F.Cu") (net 22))
 (segment (start 105.791 77.6986) (end 102.6924 74.6) (width 0.25) (layer "F.Cu") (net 22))
 (segment (start 109.78 86) (end 107.614103 86) (width 0.25) (layer "F.Cu") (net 22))
 (segment (start 111.78 83) (end 111.78 81.1476) (width 0.25) (layer "F.Cu") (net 21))
 (segment (start 102.6924 72.06) (end 102.54 72.06) (width 0.25) (layer "F.Cu") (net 21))
 (segment (start 111.78 81.1476) (end 102.6924 72.06) (width 0.25) (layer "F.Cu") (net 21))
 (segment (start 113.256 80.0836) (end 102.6924 69.52) (width 0.25) (layer "F.Cu") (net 20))
 (segment (start 113.256 83) (end 113.256 80.0836) (width 0.25) (layer "F.Cu") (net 20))
 (segment (start 102.6924 69.52) (end 102.54 69.52) (width 0.25) (layer "F.Cu") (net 20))
 (segment (start 109.78 98) (end 107.612168 98) (width 0.25) (layer "F.Cu") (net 30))
 (segment (start 107.612168 98) (end 104.532168 94.92) (width 0.25) (layer "F.Cu") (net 30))
 (segment (start 104.532168 94.92) (end 102.54 94.92) (width 0.25) (layer "F.Cu") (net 30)))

